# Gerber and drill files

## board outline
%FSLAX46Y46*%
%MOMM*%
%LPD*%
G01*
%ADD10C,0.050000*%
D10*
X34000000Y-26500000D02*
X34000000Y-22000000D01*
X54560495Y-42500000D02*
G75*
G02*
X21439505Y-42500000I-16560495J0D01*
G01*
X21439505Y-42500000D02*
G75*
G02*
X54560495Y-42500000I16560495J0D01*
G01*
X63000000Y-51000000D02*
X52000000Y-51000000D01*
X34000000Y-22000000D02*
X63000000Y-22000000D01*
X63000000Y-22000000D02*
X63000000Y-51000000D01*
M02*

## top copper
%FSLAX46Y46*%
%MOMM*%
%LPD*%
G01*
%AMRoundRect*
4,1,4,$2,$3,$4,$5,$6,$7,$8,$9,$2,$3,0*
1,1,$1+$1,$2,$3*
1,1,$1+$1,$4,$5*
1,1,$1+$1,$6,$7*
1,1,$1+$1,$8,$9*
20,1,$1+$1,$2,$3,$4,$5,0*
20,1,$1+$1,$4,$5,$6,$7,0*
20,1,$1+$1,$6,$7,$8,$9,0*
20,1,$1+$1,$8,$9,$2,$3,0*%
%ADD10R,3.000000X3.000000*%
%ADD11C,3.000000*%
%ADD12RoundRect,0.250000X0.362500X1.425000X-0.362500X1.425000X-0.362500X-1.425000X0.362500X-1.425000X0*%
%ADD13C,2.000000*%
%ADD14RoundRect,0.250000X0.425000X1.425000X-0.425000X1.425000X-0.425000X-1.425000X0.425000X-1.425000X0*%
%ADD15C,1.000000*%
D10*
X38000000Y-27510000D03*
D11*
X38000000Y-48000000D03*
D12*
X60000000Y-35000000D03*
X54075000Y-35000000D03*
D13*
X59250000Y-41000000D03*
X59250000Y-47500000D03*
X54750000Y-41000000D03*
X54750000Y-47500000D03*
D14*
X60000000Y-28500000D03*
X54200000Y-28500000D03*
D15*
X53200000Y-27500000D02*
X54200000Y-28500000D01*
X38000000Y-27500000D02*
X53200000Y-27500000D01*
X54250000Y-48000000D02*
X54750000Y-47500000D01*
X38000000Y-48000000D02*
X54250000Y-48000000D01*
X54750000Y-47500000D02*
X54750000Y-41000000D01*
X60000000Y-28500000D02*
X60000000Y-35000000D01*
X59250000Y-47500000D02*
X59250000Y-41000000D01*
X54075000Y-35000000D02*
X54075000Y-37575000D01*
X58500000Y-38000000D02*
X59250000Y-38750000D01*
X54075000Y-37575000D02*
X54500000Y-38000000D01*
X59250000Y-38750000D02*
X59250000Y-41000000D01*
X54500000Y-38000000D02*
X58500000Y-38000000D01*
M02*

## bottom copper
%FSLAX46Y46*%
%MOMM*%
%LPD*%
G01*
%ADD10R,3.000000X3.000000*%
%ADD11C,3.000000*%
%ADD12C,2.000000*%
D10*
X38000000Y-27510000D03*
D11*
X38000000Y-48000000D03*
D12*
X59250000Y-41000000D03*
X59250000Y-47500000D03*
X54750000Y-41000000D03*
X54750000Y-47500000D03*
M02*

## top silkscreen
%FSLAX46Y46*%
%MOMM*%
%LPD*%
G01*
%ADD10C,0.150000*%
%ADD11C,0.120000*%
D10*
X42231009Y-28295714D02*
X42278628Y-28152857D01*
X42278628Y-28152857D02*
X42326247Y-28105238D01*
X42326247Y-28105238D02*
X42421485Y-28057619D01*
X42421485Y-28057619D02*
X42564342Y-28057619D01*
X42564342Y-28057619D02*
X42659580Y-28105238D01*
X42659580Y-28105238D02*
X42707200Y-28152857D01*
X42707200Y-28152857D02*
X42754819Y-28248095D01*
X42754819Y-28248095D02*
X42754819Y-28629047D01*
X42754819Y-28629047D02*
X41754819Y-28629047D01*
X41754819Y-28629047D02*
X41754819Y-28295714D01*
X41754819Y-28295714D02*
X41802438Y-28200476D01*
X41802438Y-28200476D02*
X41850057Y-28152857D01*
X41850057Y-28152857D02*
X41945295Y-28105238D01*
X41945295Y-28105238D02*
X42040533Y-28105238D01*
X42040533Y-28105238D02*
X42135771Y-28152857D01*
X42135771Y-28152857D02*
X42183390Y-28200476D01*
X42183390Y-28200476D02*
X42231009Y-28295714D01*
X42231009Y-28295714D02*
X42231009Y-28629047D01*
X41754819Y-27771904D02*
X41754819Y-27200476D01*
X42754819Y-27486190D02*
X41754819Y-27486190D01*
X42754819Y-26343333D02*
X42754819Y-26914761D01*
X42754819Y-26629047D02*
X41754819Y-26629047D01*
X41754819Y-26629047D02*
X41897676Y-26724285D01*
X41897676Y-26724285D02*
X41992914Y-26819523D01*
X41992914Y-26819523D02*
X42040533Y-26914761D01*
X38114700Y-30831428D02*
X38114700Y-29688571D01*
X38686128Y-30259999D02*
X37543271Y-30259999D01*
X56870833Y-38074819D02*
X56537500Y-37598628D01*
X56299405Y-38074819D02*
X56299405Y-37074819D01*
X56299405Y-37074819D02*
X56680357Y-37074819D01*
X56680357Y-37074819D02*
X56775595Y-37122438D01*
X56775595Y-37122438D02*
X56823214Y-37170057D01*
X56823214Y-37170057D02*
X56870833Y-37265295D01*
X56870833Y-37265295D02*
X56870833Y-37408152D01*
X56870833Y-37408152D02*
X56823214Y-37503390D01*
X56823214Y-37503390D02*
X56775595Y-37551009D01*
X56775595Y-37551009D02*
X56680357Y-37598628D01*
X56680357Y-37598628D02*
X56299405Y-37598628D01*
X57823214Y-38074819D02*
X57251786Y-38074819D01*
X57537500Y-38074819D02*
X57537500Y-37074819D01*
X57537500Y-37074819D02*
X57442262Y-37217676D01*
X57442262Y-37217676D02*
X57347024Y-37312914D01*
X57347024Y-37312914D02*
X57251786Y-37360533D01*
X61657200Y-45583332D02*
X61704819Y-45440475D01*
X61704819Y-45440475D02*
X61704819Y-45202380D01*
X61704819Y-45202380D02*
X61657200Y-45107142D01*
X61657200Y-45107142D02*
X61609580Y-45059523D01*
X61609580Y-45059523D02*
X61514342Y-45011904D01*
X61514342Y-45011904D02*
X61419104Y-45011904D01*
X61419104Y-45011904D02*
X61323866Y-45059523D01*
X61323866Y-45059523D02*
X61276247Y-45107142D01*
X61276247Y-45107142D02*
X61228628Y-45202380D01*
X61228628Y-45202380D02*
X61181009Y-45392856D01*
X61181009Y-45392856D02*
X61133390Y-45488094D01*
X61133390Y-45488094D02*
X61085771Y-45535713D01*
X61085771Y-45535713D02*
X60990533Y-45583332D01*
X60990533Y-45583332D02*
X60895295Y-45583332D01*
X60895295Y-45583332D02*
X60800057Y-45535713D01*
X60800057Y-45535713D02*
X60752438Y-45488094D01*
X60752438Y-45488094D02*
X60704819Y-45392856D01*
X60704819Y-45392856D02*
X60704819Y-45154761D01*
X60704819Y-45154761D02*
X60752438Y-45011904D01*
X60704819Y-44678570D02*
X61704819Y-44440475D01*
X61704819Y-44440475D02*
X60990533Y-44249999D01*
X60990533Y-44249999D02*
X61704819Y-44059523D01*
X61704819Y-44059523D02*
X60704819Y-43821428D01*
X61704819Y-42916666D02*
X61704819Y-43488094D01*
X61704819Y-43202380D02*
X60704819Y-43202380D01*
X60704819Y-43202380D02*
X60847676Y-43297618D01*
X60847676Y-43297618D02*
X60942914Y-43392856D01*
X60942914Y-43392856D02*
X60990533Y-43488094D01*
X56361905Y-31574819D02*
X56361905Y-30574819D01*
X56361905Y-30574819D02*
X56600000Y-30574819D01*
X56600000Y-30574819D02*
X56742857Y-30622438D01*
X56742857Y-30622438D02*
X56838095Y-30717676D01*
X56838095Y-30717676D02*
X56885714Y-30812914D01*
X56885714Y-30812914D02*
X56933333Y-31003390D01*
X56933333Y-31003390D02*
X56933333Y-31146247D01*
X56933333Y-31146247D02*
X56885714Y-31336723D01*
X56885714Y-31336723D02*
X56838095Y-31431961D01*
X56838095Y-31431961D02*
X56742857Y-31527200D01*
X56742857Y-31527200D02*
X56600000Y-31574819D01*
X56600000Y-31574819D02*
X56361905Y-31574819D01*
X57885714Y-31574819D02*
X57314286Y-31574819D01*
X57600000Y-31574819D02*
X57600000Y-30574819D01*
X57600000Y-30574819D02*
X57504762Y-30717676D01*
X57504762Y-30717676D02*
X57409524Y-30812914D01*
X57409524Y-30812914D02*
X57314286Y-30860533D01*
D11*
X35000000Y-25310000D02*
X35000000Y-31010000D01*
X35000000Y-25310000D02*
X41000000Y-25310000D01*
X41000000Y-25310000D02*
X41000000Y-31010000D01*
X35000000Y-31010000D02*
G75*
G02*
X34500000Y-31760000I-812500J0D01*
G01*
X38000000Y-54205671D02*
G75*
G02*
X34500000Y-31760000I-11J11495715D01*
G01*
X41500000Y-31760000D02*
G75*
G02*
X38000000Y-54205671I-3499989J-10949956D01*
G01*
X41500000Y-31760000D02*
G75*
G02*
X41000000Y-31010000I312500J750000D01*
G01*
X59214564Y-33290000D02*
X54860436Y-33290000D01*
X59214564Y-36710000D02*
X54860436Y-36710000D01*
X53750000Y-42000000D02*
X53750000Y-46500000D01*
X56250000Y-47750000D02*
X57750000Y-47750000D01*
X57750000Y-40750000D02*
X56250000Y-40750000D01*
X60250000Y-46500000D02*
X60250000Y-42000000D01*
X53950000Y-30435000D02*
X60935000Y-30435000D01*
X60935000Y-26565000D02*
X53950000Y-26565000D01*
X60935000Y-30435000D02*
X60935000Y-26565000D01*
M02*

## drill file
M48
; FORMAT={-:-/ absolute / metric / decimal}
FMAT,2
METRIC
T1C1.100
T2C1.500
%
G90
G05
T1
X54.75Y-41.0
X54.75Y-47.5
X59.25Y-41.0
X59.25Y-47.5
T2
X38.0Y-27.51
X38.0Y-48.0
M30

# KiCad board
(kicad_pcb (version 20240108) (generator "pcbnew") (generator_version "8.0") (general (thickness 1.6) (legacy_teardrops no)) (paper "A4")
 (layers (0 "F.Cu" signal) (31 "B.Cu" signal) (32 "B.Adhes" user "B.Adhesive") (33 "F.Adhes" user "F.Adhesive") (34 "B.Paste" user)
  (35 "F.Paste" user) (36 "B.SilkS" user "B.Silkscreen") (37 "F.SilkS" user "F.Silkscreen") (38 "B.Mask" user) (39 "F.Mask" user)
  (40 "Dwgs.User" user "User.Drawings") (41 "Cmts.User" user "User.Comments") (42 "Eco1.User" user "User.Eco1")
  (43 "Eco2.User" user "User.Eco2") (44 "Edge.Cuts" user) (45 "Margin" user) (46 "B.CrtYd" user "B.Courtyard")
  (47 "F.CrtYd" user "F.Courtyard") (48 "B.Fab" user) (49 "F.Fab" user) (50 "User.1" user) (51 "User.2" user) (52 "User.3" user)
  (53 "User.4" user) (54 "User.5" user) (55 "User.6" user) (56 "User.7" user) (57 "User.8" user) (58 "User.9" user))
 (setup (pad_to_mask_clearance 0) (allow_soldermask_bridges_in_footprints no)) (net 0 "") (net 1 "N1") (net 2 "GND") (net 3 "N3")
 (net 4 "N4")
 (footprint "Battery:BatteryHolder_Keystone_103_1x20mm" (layer "F.Cu") (at 38 27.51 -90)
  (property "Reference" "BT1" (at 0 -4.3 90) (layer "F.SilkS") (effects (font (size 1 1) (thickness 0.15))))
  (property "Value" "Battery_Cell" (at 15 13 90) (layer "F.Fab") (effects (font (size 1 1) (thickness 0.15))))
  (fp_line (start -2.2 3) (end 3.5 3) (stroke (width 0.12) (type solid)) (layer "F.SilkS"))
  (fp_line (start -2.2 3) (end -2.2 -3) (stroke (width 0.12) (type solid)) (layer "F.SilkS"))
  (fp_line (start -2.2 -3) (end 3.5 -3) (stroke (width 0.12) (type solid)) (layer "F.SilkS"))
  (fp_arc (start 3.5 3) (mid 3.950694 3.136459) (end 4.25 3.5) (stroke (width 0.12) (type solid)) (layer "F.SilkS"))
  (fp_arc (start 26.695671 0) (mid 16.971103 11.358466) (end 4.25 3.5) (stroke (width 0.12) (type solid)) (layer "F.SilkS"))
  (fp_arc (start 4.25 -3.5) (mid 16.971103 -11.358466) (end 26.695671 0) (stroke (width 0.12) (type solid)) (layer "F.SilkS"))
  (fp_arc (start 4.25 -3.5) (mid 3.950694 -3.136459) (end 3.5 -3) (stroke (width 0.12) (type solid)) (layer "F.SilkS"))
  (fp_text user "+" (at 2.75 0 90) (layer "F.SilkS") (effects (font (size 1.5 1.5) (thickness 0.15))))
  (pad "1" thru_hole rect (at 0 0 270) (size 3 3) (drill 1.5) (layers "*.Cu" "*.Mask") (remove_unused_layers no) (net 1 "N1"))
  (pad "2" thru_hole circle (at 20.49 0 270) (size 3 3) (drill 1.5) (layers "*.Cu" "*.Mask") (remove_unused_layers no) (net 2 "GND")))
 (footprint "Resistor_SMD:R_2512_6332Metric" (layer "F.Cu") (at 57.0375 35 180)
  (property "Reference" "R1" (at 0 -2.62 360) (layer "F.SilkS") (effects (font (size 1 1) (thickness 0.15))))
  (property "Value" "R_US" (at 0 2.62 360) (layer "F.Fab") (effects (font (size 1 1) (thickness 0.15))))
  (fp_line (start -2.177064 1.71) (end 2.177064 1.71) (stroke (width 0.12) (type solid)) (layer "F.SilkS"))
  (fp_line (start -2.177064 -1.71) (end 2.177064 -1.71) (stroke (width 0.12) (type solid)) (layer "F.SilkS"))
  (pad "1" smd roundrect (at -2.9625 0 180) (size 1.225 3.35) (layers "F.Cu" "F.Paste" "F.Mask") (roundrect_rratio 0.204082) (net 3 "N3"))
  (pad "2" smd roundrect (at 2.9625 0 180) (size 1.225 3.35) (layers "F.Cu" "F.Paste" "F.Mask") (roundrect_rratio 0.204082) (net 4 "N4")))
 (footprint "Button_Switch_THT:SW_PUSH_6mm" (layer "F.Cu") (at 59.25 41 -90)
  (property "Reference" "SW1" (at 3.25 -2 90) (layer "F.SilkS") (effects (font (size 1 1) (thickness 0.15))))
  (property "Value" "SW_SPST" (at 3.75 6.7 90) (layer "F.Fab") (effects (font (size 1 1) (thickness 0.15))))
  (fp_line (start 1 5.5) (end 5.5 5.5) (stroke (width 0.12) (type solid)) (layer "F.SilkS"))
  (fp_line (start 6.75 3) (end 6.75 1.5) (stroke (width 0.12) (type solid)) (layer "F.SilkS"))
  (fp_line (start -0.25 1.5) (end -0.25 3) (stroke (width 0.12) (type solid)) (layer "F.SilkS"))
  (fp_line (start 5.5 -1) (end 1 -1) (stroke (width 0.12) (type solid)) (layer "F.SilkS"))
  (pad "1" thru_hole circle (at 0 0) (size 2 2) (drill 1.1) (layers "*.Cu" "*.Mask") (remove_unused_layers no) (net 4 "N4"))
  (pad "1" thru_hole circle (at 6.5 0) (size 2 2) (drill 1.1) (layers "*.Cu" "*.Mask") (remove_unused_layers no) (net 4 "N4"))
  (pad "2" thru_hole circle (at 0 4.5) (size 2 2) (drill 1.1) (layers "*.Cu" "*.Mask") (remove_unused_layers no) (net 2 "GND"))
  (pad "2" thru_hole circle (at 6.5 4.5) (size 2 2) (drill 1.1) (layers "*.Cu" "*.Mask") (remove_unused_layers no) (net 2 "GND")))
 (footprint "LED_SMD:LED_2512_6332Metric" (layer "F.Cu") (at 57.1 28.5 180)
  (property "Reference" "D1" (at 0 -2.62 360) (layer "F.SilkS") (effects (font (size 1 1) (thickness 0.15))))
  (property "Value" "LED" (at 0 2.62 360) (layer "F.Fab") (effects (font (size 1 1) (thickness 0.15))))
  (fp_line (start 3.15 -1.935) (end -3.835 -1.935) (stroke (width 0.12) (type solid)) (layer "F.SilkS"))
  (fp_line (start -3.835 1.935) (end 3.15 1.935) (stroke (width 0.12) (type solid)) (layer "F.SilkS"))
  (fp_line (start -3.835 -1.935) (end -3.835 1.935) (stroke (width 0.12) (type solid)) (layer "F.SilkS"))
  (pad "1" smd roundrect (at -2.9 0 180) (size 1.35 3.35) (layers "F.Cu" "F.Paste" "F.Mask") (roundrect_rratio 0.185185) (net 3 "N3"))
  (pad "2" smd roundrect (at 2.9 0 180) (size 1.35 3.35) (layers "F.Cu" "F.Paste" "F.Mask") (roundrect_rratio 0.185185) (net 1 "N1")))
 (gr_line (start 34 26.5) (end 34 22) (stroke (width 0.05) (type default)) (layer "Edge.Cuts"))
 (gr_circle (center 38 42.5) (end 52.5 34.5) (stroke (width 0.05) (type default)) (fill none) (layer "Edge.Cuts"))
 (gr_line (start 63 51) (end 52 51) (stroke (width 0.05) (type default)) (layer "Edge.Cuts"))
 (gr_line (start 34 22) (end 63 22) (stroke (width 0.05) (type default)) (layer "Edge.Cuts"))
 (gr_line (start 63 22) (end 63 51) (stroke (width 0.05) (type default)) (layer "Edge.Cuts"))
 (segment (start 53.2 27.5) (end 54.2 28.5) (width 1) (layer "F.Cu") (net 1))
 (segment (start 38 27.5) (end 53.2 27.5) (width 1) (layer "F.Cu") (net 1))
 (segment (start 54.25 48) (end 54.75 47.5) (width 1) (layer "F.Cu") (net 2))
 (segment (start 38 48) (end 54.25 48) (width 1) (layer "F.Cu") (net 2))
 (segment (start 54.75 47.5) (end 54.75 41) (width 1) (layer "F.Cu") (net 2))
 (segment (start 60 28.5) (end 60 35) (width 1) (layer "F.Cu") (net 3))
 (segment (start 59.25 47.5) (end 59.25 41) (width 1) (layer "F.Cu") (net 4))
 (segment (start 54.075 35) (end 54.075 37.575) (width 1) (layer "F.Cu") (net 4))
 (segment (start 58.5 38) (end 59.25 38.75) (width 1) (layer "F.Cu") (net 4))
 (segment (start 54.075 37.575) (end 54.5 38) (width 1) (layer "F.Cu") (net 4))
 (segment (start 59.25 38.75) (end 59.25 41) (width 1) (layer "F.Cu") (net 4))
 (segment (start 54.5 38) (end 58.5 38) (width 1) (layer "F.Cu") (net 4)))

